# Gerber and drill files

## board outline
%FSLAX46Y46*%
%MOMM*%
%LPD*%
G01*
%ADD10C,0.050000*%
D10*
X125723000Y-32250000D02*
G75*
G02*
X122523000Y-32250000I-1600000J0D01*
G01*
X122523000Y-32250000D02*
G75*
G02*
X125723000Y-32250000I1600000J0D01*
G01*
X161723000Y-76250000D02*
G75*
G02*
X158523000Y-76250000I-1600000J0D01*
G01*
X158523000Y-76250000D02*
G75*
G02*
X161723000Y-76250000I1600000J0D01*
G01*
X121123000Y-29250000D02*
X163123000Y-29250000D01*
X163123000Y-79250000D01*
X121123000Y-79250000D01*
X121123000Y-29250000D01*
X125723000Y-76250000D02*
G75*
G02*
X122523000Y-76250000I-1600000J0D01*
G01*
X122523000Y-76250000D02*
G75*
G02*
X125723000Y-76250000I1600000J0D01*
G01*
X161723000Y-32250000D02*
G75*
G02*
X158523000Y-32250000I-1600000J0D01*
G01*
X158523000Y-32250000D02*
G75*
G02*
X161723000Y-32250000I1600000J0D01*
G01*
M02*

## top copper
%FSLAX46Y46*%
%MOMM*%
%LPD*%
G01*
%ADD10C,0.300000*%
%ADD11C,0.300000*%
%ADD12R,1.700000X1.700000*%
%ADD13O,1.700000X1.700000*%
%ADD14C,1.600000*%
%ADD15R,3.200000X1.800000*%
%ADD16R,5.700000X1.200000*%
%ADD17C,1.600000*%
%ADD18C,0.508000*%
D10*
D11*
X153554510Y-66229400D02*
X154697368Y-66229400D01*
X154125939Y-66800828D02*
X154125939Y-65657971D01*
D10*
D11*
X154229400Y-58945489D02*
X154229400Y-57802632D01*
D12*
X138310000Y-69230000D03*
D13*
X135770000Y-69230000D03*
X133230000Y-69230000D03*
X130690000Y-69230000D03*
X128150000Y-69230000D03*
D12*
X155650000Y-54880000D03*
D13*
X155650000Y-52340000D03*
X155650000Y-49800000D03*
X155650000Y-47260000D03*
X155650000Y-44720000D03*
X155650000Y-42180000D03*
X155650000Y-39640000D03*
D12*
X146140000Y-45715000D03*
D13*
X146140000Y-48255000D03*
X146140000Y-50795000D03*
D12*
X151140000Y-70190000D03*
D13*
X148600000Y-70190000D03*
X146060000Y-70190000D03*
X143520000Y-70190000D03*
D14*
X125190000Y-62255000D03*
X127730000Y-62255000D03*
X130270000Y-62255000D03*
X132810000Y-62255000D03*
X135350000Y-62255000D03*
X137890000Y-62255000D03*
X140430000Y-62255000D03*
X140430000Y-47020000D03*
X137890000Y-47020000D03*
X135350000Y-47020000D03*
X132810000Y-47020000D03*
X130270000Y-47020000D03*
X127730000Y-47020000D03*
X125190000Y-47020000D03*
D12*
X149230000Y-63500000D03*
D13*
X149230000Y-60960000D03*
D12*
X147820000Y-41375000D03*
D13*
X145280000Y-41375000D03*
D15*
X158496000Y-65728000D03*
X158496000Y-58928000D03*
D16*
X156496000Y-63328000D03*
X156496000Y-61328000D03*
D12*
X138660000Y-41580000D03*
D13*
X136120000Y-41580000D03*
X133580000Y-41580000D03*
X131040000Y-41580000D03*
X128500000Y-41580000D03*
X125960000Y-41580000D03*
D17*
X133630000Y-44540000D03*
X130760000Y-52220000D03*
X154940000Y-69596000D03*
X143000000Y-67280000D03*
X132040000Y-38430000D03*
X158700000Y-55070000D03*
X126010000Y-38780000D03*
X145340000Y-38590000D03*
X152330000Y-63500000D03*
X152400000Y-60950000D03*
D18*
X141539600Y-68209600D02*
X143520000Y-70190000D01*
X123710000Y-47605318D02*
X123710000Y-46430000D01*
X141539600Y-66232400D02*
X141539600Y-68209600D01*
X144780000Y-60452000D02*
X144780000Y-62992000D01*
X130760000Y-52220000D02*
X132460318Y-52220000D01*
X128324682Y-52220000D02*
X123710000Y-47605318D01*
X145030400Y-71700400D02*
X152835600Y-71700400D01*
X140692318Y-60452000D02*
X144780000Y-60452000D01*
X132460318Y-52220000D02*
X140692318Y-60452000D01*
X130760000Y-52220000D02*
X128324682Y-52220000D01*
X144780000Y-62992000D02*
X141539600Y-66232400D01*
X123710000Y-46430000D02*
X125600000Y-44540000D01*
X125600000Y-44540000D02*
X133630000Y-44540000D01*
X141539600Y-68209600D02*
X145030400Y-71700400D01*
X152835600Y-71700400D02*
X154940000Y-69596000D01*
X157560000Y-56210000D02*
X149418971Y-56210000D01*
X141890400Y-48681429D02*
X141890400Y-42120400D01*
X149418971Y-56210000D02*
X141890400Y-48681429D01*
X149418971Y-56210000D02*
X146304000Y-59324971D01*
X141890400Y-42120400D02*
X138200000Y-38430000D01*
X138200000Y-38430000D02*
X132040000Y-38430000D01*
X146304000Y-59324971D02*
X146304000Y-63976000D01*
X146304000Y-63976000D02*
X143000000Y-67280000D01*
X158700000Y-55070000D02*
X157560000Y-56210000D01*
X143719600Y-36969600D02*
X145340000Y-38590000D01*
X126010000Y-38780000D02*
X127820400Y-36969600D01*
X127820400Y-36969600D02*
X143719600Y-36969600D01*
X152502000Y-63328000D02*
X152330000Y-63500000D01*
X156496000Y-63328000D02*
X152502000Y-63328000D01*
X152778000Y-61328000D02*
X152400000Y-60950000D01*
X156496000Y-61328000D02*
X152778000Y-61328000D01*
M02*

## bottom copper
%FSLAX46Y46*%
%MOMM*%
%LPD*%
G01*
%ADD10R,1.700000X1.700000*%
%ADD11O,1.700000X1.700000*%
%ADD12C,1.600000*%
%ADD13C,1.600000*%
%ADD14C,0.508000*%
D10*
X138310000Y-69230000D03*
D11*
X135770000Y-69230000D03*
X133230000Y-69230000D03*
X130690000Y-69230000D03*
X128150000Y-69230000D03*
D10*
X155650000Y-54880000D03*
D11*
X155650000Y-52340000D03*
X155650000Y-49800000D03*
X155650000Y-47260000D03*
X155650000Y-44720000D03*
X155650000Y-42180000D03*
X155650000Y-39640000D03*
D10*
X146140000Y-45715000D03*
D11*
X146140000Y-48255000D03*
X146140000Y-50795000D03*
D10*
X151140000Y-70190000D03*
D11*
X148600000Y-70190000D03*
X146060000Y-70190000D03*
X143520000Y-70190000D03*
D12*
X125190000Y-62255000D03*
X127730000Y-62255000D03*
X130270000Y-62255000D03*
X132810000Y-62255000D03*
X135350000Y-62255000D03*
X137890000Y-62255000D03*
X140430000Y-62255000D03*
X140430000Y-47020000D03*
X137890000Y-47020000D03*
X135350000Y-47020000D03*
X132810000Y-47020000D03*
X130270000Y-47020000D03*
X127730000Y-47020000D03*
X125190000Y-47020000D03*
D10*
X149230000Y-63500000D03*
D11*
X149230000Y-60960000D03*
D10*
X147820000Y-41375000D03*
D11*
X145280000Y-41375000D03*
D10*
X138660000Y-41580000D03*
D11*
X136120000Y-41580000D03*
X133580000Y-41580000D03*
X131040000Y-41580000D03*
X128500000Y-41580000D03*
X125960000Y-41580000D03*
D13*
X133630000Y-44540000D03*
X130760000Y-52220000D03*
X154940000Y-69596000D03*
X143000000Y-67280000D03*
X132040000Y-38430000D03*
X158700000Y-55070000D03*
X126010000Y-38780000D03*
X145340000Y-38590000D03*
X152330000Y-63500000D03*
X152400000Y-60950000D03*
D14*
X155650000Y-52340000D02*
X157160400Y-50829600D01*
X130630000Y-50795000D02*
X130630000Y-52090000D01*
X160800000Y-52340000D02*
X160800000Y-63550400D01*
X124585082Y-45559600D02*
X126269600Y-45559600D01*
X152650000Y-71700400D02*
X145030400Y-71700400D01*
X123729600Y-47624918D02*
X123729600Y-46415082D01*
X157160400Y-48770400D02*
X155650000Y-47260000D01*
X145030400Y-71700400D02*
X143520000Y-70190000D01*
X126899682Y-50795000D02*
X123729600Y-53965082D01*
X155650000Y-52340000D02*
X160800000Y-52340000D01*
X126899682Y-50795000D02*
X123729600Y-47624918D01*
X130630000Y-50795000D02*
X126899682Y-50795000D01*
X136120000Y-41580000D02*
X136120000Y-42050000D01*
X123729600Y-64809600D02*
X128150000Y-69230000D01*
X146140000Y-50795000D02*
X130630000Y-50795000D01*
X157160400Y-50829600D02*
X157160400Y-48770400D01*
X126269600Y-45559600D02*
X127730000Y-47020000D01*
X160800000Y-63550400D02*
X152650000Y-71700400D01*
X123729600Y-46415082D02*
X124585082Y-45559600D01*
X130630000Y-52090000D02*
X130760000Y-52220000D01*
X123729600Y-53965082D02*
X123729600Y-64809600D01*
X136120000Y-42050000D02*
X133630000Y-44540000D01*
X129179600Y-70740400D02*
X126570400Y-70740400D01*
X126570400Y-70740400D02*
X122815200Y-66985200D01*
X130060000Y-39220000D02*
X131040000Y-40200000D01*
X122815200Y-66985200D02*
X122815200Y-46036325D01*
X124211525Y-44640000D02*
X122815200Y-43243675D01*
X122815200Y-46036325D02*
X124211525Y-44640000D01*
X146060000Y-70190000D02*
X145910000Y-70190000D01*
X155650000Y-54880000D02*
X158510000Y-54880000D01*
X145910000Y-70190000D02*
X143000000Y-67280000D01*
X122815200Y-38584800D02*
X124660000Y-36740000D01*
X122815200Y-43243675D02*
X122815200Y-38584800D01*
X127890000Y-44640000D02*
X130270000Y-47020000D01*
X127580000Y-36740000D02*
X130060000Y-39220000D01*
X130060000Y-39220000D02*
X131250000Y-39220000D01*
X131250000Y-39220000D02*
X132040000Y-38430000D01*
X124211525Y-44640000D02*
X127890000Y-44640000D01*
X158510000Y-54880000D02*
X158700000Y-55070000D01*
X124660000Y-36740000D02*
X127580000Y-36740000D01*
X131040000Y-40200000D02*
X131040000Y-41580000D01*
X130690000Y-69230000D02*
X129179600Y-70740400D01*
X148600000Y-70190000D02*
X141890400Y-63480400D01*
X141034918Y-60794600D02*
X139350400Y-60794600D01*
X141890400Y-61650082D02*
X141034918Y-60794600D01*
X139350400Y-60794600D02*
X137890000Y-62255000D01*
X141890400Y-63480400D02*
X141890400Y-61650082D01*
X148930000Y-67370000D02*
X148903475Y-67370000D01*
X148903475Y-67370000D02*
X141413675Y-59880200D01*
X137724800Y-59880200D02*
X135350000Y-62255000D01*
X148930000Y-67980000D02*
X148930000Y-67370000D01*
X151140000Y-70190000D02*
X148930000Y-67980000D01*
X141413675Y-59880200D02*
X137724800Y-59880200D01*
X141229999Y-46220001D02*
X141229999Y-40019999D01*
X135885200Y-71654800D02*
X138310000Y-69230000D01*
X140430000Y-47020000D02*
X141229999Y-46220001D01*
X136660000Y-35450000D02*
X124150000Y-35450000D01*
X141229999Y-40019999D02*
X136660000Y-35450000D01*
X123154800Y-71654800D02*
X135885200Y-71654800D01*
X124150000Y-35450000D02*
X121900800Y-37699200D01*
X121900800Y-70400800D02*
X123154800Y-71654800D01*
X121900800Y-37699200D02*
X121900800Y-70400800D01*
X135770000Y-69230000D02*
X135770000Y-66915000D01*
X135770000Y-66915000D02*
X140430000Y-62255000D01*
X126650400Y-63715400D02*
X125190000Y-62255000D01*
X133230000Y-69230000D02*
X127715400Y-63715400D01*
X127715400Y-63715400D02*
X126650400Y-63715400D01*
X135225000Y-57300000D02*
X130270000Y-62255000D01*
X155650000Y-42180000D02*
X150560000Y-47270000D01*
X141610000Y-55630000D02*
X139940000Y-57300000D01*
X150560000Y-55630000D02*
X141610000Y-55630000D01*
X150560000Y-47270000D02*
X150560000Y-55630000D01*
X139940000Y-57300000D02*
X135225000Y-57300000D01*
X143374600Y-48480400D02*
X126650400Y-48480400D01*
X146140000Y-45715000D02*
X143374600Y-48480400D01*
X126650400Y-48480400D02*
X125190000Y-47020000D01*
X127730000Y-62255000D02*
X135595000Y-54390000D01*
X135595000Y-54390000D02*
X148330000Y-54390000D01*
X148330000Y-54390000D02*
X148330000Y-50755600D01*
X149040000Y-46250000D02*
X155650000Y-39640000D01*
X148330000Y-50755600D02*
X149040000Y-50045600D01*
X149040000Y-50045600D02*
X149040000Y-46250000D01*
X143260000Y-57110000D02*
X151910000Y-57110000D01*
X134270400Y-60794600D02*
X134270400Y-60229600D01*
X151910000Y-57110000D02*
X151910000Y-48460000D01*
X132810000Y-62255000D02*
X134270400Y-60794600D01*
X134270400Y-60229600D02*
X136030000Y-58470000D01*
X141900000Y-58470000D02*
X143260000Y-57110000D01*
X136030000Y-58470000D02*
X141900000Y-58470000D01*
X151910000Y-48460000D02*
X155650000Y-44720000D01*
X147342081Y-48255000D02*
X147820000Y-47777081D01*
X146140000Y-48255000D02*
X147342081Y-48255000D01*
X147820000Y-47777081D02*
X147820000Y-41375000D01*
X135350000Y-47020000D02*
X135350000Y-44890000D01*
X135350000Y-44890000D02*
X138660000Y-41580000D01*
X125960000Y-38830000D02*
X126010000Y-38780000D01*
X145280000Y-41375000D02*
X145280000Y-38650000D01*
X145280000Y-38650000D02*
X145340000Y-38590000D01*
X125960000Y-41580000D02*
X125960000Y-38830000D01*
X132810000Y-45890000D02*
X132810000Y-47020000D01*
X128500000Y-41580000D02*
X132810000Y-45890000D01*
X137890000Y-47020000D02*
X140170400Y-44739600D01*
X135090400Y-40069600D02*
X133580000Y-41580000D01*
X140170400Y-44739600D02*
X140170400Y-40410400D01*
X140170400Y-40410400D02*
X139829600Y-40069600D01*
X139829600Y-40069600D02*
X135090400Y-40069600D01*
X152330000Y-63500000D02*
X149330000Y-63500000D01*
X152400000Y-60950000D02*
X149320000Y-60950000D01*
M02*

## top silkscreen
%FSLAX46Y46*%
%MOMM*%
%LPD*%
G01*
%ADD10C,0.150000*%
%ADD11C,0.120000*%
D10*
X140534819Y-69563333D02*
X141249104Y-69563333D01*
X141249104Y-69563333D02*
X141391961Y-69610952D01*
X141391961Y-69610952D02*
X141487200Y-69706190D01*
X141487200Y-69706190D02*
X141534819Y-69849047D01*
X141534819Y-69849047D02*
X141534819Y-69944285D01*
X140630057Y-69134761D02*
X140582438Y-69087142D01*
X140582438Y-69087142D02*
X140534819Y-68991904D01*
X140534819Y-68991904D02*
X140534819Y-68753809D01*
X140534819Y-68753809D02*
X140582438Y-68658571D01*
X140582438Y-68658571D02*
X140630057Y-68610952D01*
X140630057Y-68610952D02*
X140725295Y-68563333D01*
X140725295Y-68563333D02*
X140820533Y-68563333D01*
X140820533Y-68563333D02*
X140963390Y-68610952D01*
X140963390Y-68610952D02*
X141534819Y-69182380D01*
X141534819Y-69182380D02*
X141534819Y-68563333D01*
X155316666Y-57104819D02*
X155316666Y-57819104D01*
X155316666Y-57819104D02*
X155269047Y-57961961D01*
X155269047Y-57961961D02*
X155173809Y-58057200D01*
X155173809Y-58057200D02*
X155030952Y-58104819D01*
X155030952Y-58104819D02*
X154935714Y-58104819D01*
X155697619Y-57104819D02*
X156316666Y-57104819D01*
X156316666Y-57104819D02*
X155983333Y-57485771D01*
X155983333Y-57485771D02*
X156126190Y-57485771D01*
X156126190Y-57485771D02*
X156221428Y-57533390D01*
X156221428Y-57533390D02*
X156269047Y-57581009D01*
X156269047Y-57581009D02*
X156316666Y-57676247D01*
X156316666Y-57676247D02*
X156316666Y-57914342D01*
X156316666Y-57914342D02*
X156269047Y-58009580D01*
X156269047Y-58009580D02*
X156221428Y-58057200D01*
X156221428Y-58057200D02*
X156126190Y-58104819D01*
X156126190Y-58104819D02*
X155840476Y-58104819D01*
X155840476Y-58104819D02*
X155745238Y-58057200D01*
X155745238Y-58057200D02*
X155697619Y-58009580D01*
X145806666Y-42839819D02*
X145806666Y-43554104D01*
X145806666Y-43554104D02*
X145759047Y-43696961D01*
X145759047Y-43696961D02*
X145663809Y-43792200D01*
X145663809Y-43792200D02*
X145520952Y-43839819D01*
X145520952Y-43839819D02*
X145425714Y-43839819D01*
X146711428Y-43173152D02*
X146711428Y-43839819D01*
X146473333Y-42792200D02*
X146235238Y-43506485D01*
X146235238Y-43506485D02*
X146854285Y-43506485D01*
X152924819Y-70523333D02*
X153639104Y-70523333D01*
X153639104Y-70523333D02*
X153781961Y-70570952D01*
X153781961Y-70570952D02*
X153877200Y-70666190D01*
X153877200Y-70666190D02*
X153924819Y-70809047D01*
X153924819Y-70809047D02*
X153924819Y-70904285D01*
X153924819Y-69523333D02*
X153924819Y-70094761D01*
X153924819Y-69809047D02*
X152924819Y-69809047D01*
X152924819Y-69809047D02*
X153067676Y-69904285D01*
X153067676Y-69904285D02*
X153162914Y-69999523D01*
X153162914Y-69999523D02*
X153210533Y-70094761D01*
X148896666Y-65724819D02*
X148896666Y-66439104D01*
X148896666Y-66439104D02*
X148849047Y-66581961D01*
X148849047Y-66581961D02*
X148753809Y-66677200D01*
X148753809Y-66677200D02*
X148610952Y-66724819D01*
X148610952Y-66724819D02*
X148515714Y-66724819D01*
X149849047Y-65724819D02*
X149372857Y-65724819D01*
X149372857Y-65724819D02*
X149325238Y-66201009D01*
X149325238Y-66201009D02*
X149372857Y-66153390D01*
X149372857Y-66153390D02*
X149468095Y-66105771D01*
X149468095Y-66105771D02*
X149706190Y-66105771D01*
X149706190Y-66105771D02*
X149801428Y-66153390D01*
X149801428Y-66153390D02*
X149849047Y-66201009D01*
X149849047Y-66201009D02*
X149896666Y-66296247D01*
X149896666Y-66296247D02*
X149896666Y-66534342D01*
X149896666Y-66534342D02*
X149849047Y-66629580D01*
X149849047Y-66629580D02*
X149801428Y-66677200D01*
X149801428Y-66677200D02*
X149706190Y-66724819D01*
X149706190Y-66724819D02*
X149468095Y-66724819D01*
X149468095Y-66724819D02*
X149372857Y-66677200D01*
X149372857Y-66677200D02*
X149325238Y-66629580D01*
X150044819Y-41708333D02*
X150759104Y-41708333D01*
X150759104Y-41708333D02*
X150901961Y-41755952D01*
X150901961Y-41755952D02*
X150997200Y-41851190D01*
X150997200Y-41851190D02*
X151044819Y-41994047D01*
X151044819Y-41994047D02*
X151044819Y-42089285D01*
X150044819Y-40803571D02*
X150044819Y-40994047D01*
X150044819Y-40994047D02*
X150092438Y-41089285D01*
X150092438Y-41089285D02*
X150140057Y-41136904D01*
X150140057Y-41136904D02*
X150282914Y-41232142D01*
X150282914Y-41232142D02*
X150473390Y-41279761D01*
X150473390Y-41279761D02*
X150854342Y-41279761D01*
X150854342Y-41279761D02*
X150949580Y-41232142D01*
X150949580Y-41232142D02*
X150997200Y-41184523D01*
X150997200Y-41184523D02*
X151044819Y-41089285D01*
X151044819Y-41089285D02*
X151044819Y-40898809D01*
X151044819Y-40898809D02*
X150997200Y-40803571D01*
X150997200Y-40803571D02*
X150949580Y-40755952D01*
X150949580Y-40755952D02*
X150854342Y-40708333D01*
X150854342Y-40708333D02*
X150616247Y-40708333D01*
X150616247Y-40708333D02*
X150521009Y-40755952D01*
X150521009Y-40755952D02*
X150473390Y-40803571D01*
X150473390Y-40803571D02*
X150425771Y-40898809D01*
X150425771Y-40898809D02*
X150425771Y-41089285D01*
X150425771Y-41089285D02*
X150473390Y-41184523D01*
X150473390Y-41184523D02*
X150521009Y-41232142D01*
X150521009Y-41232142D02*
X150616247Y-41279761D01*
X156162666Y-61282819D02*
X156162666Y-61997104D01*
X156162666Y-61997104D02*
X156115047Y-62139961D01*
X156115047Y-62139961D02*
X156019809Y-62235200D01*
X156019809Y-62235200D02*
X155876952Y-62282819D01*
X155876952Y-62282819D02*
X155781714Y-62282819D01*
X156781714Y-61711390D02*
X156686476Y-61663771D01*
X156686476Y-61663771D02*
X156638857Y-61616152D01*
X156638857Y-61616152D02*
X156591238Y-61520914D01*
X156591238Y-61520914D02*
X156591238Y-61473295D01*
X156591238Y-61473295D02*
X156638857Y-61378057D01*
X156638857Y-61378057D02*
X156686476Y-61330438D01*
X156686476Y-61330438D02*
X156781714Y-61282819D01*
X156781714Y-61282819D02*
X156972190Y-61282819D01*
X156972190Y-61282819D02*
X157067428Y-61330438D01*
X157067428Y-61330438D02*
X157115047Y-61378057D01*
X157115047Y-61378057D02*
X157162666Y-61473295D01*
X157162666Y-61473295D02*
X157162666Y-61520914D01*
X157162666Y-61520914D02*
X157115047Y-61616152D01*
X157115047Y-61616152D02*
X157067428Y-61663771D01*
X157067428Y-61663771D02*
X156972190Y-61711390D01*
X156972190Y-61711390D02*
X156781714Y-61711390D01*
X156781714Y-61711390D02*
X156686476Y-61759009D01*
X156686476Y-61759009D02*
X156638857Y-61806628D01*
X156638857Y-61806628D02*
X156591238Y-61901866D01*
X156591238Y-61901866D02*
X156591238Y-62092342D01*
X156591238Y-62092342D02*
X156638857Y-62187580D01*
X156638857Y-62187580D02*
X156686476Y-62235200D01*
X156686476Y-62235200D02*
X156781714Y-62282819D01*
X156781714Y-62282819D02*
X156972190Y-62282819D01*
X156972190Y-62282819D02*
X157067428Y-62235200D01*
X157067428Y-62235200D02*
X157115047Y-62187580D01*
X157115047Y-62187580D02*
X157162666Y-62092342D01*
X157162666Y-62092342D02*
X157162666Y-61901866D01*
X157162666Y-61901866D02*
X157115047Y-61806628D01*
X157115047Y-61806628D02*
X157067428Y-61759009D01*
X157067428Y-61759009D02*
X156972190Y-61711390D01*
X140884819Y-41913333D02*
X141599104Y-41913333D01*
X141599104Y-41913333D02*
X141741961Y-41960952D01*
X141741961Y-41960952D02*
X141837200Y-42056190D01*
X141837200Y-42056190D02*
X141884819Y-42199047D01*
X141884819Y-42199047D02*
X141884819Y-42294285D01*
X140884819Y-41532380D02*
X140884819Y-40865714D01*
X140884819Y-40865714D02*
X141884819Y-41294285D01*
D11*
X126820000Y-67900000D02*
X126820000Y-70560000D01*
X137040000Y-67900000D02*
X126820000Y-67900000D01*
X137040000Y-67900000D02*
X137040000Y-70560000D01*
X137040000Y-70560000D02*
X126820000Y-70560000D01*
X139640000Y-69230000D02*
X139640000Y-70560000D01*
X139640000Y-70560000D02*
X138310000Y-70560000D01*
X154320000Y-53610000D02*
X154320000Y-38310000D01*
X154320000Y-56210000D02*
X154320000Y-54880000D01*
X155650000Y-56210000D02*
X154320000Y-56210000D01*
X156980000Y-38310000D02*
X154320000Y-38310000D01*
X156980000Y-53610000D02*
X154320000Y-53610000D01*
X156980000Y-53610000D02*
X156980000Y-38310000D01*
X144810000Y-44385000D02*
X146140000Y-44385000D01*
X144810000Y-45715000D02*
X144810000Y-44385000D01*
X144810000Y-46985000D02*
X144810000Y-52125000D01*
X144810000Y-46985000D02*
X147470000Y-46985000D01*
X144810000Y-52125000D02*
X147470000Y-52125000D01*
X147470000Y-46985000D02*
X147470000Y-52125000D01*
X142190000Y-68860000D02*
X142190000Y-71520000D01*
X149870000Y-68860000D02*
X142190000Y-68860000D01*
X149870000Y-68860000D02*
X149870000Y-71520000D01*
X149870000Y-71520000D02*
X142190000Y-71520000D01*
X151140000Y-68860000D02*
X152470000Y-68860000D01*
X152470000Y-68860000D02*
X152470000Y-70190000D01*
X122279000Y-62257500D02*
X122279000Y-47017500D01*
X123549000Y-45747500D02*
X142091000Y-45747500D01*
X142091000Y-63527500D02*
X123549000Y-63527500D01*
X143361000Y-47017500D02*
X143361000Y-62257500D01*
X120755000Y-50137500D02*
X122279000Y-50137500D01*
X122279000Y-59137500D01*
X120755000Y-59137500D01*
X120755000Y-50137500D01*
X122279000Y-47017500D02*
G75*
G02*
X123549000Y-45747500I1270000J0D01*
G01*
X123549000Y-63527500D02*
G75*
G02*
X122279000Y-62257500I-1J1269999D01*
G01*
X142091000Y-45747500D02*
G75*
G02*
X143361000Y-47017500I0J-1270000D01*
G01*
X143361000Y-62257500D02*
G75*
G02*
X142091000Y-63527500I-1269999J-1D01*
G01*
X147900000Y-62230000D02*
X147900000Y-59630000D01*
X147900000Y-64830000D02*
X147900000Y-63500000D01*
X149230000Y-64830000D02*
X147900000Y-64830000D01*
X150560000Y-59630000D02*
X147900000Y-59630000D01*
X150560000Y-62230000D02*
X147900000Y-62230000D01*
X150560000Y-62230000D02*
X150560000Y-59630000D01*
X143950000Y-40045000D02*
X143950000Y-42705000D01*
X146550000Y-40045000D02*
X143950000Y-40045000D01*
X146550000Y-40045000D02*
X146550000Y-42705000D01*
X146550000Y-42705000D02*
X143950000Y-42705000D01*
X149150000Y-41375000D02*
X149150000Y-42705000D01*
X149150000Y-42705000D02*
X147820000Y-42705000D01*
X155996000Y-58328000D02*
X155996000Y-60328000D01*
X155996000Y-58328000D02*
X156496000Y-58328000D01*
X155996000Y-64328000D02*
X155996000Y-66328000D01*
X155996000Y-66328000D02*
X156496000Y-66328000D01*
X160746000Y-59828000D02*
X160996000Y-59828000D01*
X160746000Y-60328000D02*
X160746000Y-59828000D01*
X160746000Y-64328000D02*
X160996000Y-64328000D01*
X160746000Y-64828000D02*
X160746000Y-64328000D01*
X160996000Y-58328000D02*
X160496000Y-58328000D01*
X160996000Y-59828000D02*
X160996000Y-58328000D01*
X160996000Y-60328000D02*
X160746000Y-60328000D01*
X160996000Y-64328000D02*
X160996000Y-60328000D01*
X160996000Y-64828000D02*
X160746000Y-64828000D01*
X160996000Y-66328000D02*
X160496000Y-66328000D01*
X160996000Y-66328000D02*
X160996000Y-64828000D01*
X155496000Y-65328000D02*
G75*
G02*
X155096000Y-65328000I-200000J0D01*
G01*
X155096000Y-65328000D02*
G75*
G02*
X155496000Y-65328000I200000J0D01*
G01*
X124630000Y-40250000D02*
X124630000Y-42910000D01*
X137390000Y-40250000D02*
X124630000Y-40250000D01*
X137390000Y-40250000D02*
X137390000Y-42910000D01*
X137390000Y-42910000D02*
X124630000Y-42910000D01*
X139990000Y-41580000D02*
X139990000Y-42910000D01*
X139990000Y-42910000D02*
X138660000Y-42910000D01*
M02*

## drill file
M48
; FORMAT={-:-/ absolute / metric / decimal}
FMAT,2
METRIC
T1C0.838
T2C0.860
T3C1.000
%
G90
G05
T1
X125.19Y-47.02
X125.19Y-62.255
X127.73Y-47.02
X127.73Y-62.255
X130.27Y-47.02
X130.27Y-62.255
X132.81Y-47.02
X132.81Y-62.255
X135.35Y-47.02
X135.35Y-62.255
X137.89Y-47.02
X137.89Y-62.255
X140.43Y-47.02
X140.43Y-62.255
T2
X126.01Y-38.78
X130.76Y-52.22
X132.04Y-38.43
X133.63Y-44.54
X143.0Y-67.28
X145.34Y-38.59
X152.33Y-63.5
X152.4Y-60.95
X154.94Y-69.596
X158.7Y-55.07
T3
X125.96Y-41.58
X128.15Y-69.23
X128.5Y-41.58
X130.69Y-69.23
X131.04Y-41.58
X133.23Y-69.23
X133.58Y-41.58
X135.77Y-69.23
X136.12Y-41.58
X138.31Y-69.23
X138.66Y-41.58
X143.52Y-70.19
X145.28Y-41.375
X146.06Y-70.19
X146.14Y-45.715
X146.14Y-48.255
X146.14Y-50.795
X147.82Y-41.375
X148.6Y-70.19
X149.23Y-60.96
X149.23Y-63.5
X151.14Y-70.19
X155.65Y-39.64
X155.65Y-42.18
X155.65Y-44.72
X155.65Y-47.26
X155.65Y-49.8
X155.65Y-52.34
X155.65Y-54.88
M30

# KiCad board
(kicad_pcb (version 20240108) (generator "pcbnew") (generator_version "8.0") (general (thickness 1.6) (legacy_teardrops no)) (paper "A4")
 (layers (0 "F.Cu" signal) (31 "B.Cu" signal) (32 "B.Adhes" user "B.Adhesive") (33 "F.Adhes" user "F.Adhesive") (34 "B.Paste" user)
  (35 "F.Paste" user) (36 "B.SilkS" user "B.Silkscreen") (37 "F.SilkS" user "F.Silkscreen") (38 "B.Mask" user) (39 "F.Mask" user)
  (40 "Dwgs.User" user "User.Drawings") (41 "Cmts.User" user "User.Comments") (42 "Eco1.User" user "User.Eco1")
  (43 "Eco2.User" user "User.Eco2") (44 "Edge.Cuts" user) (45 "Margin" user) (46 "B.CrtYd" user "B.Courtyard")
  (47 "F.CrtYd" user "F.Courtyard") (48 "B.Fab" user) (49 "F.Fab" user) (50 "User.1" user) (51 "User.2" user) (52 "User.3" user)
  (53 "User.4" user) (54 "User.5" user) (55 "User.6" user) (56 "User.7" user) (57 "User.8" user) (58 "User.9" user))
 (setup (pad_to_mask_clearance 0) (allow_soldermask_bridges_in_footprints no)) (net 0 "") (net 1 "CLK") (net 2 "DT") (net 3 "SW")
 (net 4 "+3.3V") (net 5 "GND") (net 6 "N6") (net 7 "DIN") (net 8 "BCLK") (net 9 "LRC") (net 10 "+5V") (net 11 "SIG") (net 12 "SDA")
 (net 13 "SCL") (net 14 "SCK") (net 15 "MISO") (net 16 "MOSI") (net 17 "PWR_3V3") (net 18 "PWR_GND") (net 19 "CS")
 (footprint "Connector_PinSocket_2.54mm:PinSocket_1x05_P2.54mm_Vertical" (layer "F.Cu") (at 138.31 69.23 -90)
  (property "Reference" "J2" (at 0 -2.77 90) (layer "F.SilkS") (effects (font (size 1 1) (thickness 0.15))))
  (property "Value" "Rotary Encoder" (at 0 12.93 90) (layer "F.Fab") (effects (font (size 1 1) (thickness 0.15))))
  (fp_line (start -1.33 11.49) (end 1.33 11.49) (stroke (width 0.12) (type solid)) (layer "F.SilkS"))
  (fp_line (start -1.33 1.27) (end -1.33 11.49) (stroke (width 0.12) (type solid)) (layer "F.SilkS"))
  (fp_line (start -1.33 1.27) (end 1.33 1.27) (stroke (width 0.12) (type solid)) (layer "F.SilkS"))
  (fp_line (start 1.33 1.27) (end 1.33 11.49) (stroke (width 0.12) (type solid)) (layer "F.SilkS"))
  (fp_line (start 0 -1.33) (end 1.33 -1.33) (stroke (width 0.12) (type solid)) (layer "F.SilkS"))
  (fp_line (start 1.33 -1.33) (end 1.33 0) (stroke (width 0.12) (type solid)) (layer "F.SilkS"))
  (pad "1" thru_hole rect (at 0 0 270) (size 1.7 1.7) (drill 1) (layers "*.Cu" "*.Mask") (remove_unused_layers no) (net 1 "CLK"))
  (pad "2" thru_hole oval (at 0 2.54 270) (size 1.7 1.7) (drill 1) (layers "*.Cu" "*.Mask") (remove_unused_layers no) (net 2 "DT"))
  (pad "3" thru_hole oval (at 0 5.08 270) (size 1.7 1.7) (drill 1) (layers "*.Cu" "*.Mask") (remove_unused_layers no) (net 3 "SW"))
  (pad "4" thru_hole oval (at 0 7.62 270) (size 1.7 1.7) (drill 1) (layers "*.Cu" "*.Mask") (remove_unused_layers no) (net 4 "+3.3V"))
  (pad "5" thru_hole oval (at 0 10.16 270) (size 1.7 1.7) (drill 1) (layers "*.Cu" "*.Mask") (remove_unused_layers no) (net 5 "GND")))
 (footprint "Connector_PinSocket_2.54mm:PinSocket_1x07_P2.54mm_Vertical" (layer "F.Cu") (at 155.65 54.88 180)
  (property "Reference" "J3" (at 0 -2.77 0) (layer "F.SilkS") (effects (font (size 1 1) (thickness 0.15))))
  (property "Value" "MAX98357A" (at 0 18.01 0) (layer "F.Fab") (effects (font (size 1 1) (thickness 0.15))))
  (fp_line (start 1.33 1.27) (end 1.33 16.57) (stroke (width 0.12) (type solid)) (layer "F.SilkS"))
  (fp_line (start 1.33 -1.33) (end 1.33 0) (stroke (width 0.12) (type solid)) (layer "F.SilkS"))
  (fp_line (start 0 -1.33) (end 1.33 -1.33) (stroke (width 0.12) (type solid)) (layer "F.SilkS"))
  (fp_line (start -1.33 16.57) (end 1.33 16.57) (stroke (width 0.12) (type solid)) (layer "F.SilkS"))
  (fp_line (start -1.33 1.27) (end 1.33 1.27) (stroke (width 0.12) (type solid)) (layer "F.SilkS"))
  (fp_line (start -1.33 1.27) (end -1.33 16.57) (stroke (width 0.12) (type solid)) (layer "F.SilkS"))
  (pad "1" thru_hole rect (at 0 0 180) (size 1.7 1.7) (drill 1) (layers "*.Cu" "*.Mask") (remove_unused_layers no) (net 4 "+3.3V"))
  (pad "2" thru_hole oval (at 0 2.54 180) (size 1.7 1.7) (drill 1) (layers "*.Cu" "*.Mask") (remove_unused_layers no) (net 5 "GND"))
  (pad "3" thru_hole oval (at 0 5.08 180) (size 1.7 1.7) (drill 1) (layers "*.Cu" "*.Mask") (remove_unused_layers no) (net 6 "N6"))
  (pad "4" thru_hole oval (at 0 7.62 180) (size 1.7 1.7) (drill 1) (layers "*.Cu" "*.Mask") (remove_unused_layers no) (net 5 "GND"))
  (pad "5" thru_hole oval (at 0 10.16 180) (size 1.7 1.7) (drill 1) (layers "*.Cu" "*.Mask") (remove_unused_layers no) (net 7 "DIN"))
  (pad "6" thru_hole oval (at 0 12.7 180) (size 1.7 1.7) (drill 1) (layers "*.Cu" "*.Mask") (remove_unused_layers no) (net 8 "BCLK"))
  (pad "7" thru_hole oval (at 0 15.24 180) (size 1.7 1.7) (drill 1) (layers "*.Cu" "*.Mask") (remove_unused_layers no) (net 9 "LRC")))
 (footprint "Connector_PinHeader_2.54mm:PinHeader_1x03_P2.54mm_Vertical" (layer "F.Cu") (at 146.14 45.715)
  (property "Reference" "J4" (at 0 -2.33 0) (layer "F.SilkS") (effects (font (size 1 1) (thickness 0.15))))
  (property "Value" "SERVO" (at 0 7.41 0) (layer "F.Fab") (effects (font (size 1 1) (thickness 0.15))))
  (fp_line (start -1.33 -1.33) (end 0 -1.33) (stroke (width 0.12) (type solid)) (layer "F.SilkS"))
  (fp_line (start -1.33 0) (end -1.33 -1.33) (stroke (width 0.12) (type solid)) (layer "F.SilkS"))
  (fp_line (start -1.33 1.27) (end -1.33 6.41) (stroke (width 0.12) (type solid)) (layer "F.SilkS"))
  (fp_line (start -1.33 1.27) (end 1.33 1.27) (stroke (width 0.12) (type solid)) (layer "F.SilkS"))
  (fp_line (start -1.33 6.41) (end 1.33 6.41) (stroke (width 0.12) (type solid)) (layer "F.SilkS"))
  (fp_line (start 1.33 1.27) (end 1.33 6.41) (stroke (width 0.12) (type solid)) (layer "F.SilkS"))
  (pad "1" thru_hole rect (at 0 0) (size 1.7 1.7) (drill 1) (layers "*.Cu" "*.Mask") (remove_unused_layers no) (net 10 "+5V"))
  (pad "2" thru_hole oval (at 0 2.54) (size 1.7 1.7) (drill 1) (layers "*.Cu" "*.Mask") (remove_unused_layers no) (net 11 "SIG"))
  (pad "3" thru_hole oval (at 0 5.08) (size 1.7 1.7) (drill 1) (layers "*.Cu" "*.Mask") (remove_unused_layers no) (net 5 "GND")))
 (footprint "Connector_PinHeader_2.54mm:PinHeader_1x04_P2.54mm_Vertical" (layer "F.Cu") (at 151.14 70.19 -90)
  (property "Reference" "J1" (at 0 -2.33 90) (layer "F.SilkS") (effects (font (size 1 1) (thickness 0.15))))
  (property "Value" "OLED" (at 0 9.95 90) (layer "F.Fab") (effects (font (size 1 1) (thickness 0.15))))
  (fp_line (start -1.33 8.95) (end 1.33 8.95) (stroke (width 0.12) (type solid)) (layer "F.SilkS"))
  (fp_line (start -1.33 1.27) (end -1.33 8.95) (stroke (width 0.12) (type solid)) (layer "F.SilkS"))
  (fp_line (start -1.33 1.27) (end 1.33 1.27) (stroke (width 0.12) (type solid)) (layer "F.SilkS"))
  (fp_line (start 1.33 1.27) (end 1.33 8.95) (stroke (width 0.12) (type solid)) (layer "F.SilkS"))
  (fp_line (start -1.33 0) (end -1.33 -1.33) (stroke (width 0.12) (type solid)) (layer "F.SilkS"))
  (fp_line (start -1.33 -1.33) (end 0 -1.33) (stroke (width 0.12) (type solid)) (layer "F.SilkS"))
  (pad "1" thru_hole rect (at 0 0 270) (size 1.7 1.7) (drill 1) (layers "*.Cu" "*.Mask") (remove_unused_layers no) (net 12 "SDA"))
  (pad "2" thru_hole oval (at 0 2.54 270) (size 1.7 1.7) (drill 1) (layers "*.Cu" "*.Mask") (remove_unused_layers no) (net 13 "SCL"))
  (pad "3" thru_hole oval (at 0 5.08 270) (size 1.7 1.7) (drill 1) (layers "*.Cu" "*.Mask") (remove_unused_layers no) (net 4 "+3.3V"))
  (pad "4" thru_hole oval (at 0 7.62 270) (size 1.7 1.7) (drill 1) (layers "*.Cu" "*.Mask") (remove_unused_layers no) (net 5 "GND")))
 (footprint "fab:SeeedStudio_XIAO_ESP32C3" (layer "F.Cu") (at 132.81 54.64 90)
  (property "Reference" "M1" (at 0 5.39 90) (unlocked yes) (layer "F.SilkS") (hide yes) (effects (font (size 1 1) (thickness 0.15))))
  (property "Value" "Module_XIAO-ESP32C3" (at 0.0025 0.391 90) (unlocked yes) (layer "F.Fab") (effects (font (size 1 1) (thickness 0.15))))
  (fp_line (start -7.6175 -10.531) (end 7.6225 -10.531) (stroke (width 0.12) (type solid)) (layer "F.SilkS"))
  (fp_line (start 8.8925 -9.261) (end 8.8925 9.281) (stroke (width 0.12) (type solid)) (layer "F.SilkS"))
  (fp_line (start -8.8875 9.281) (end -8.8875 -9.261) (stroke (width 0.12) (type solid)) (layer "F.SilkS"))
  (fp_line (start 7.6225 10.551) (end -7.6175 10.551) (stroke (width 0.12) (type solid)) (layer "F.SilkS"))
  (fp_rect (start -4.4975 -10.531) (end 4.5025 -12.055) (stroke (width 0.12) (type solid)) (fill none) (layer "F.SilkS"))
  (fp_arc (start 7.6225 -10.531) (mid 8.520526 -10.159026) (end 8.8925 -9.261) (stroke (width 0.12) (type solid)) (layer "F.SilkS"))
  (fp_arc (start -8.8875 -9.261) (mid -8.515526 -10.159026) (end -7.6175 -10.531) (stroke (width 0.12) (type solid)) (layer "F.SilkS"))
  (fp_arc (start 8.8925 9.281) (mid 8.520526 10.179026) (end 7.6225 10.551) (stroke (width 0.12) (type solid)) (layer "F.SilkS"))
  (fp_arc (start -7.6175 10.551) (mid -8.515526 10.179026) (end -8.8875 9.281) (stroke (width 0.12) (type solid)) (layer "F.SilkS"))
  (pad "1" thru_hole circle (at -7.615 -7.62 90) (size 1.6 1.6) (drill 0.8382) (layers "*.Cu" "*.Mask") (remove_unused_layers no)
   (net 3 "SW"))
  (pad "2" thru_hole circle (at -7.615 -5.08 90) (size 1.6 1.6) (drill 0.8382) (layers "*.Cu" "*.Mask") (remove_unused_layers no)
   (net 9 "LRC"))
  (pad "3" thru_hole circle (at -7.615 -2.54 90) (size 1.6 1.6) (drill 0.8382) (layers "*.Cu" "*.Mask") (remove_unused_layers no)
   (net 8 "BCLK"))
  (pad "4" thru_hole circle (at -7.615 0 90) (size 1.6 1.6) (drill 0.8382) (layers "*.Cu" "*.Mask") (remove_unused_layers no) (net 7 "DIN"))
  (pad "5" thru_hole circle (at -7.615 2.54 90) (size 1.6 1.6) (drill 0.8382) (layers "*.Cu" "*.Mask") (remove_unused_layers no)
   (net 12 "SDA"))
  (pad "6" thru_hole circle (at -7.615 5.08 90) (size 1.6 1.6) (drill 0.8382) (layers "*.Cu" "*.Mask") (remove_unused_layers no)
   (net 13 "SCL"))
  (pad "7" thru_hole circle (at -7.615 7.62 90) (size 1.6 1.6) (drill 0.8382) (layers "*.Cu" "*.Mask") (remove_unused_layers no)
   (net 2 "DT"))
  (pad "8" thru_hole circle (at 7.62 7.62 90) (size 1.6 1.6) (drill 0.8382) (layers "*.Cu" "*.Mask") (remove_unused_layers no) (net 1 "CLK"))
  (pad "9" thru_hole circle (at 7.62 5.08 90) (size 1.6 1.6) (drill 0.8382) (layers "*.Cu" "*.Mask") (remove_unused_layers no)
   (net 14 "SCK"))
  (pad "10" thru_hole circle (at 7.62 2.54 90) (size 1.6 1.6) (drill 0.8382) (layers "*.Cu" "*.Mask") (remove_unused_layers no)
   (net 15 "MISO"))
  (pad "11" thru_hole circle (at 7.62 0 90) (size 1.6 1.6) (drill 0.8382) (layers "*.Cu" "*.Mask") (remove_unused_layers no) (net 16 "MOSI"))
  (pad "12" thru_hole circle (at 7.62 -2.54 90) (size 1.6 1.6) (drill 0.8382) (layers "*.Cu" "*.Mask") (remove_unused_layers no)
   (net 4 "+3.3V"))
  (pad "13" thru_hole circle (at 7.62 -5.08 90) (size 1.6 1.6) (drill 0.8382) (layers "*.Cu" "*.Mask") (remove_unused_layers no)
   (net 5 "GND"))
  (pad "14" thru_hole circle (at 7.62 -7.62 90) (size 1.6 1.6) (drill 0.8382) (layers "*.Cu" "*.Mask") (remove_unused_layers no)
   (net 10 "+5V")))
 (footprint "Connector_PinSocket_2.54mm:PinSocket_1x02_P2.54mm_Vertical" (layer "F.Cu") (at 149.23 63.5 180)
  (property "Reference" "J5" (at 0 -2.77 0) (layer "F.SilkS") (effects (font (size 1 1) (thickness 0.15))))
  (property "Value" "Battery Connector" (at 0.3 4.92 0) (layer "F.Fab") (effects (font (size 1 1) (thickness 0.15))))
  (fp_line (start 1.33 1.27) (end 1.33 3.87) (stroke (width 0.12) (type solid)) (layer "F.SilkS"))
  (fp_line (start 1.33 -1.33) (end 1.33 0) (stroke (width 0.12) (type solid)) (layer "F.SilkS"))
  (fp_line (start 0 -1.33) (end 1.33 -1.33) (stroke (width 0.12) (type solid)) (layer "F.SilkS"))
  (fp_line (start -1.33 3.87) (end 1.33 3.87) (stroke (width 0.12) (type solid)) (layer "F.SilkS"))
  (fp_line (start -1.33 1.27) (end 1.33 1.27) (stroke (width 0.12) (type solid)) (layer "F.SilkS"))
  (fp_line (start -1.33 1.27) (end -1.33 3.87) (stroke (width 0.12) (type solid)) (layer "F.SilkS"))
  (pad "1" thru_hole rect (at 0 0 180) (size 1.7 1.7) (drill 1) (layers "*.Cu" "*.Mask") (remove_unused_layers no) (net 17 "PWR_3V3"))
  (pad "2" thru_hole oval (at 0 2.54 180) (size 1.7 1.7) (drill 1) (layers "*.Cu" "*.Mask") (remove_unused_layers no) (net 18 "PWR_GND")))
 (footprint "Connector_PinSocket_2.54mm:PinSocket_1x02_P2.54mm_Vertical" (layer "F.Cu") (at 147.82 41.375 -90)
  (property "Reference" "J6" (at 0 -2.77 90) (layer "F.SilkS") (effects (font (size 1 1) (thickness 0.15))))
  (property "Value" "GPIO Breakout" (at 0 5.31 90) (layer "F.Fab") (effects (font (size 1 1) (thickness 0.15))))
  (fp_line (start -1.33 3.87) (end 1.33 3.87) (stroke (width 0.12) (type solid)) (layer "F.SilkS"))
  (fp_line (start -1.33 1.27) (end -1.33 3.87) (stroke (width 0.12) (type solid)) (layer "F.SilkS"))
  (fp_line (start -1.33 1.27) (end 1.33 1.27) (stroke (width 0.12) (type solid)) (layer "F.SilkS"))
  (fp_line (start 1.33 1.27) (end 1.33 3.87) (stroke (width 0.12) (type solid)) (layer "F.SilkS"))
  (fp_line (start 0 -1.33) (end 1.33 -1.33) (stroke (width 0.12) (type solid)) (layer "F.SilkS"))
  (fp_line (start 1.33 -1.33) (end 1.33 0) (stroke (width 0.12) (type solid)) (layer "F.SilkS"))
  (pad "1" thru_hole rect (at 0 0 270) (size 1.7 1.7) (drill 1) (layers "*.Cu" "*.Mask") (remove_unused_layers no) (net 11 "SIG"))
  (pad "2" thru_hole oval (at 0 2.54 270) (size 1.7 1.7) (drill 1) (layers "*.Cu" "*.Mask") (remove_unused_layers no) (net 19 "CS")))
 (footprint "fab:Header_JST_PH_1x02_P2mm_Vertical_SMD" (layer "F.Cu") (at 156.496 62.328 180)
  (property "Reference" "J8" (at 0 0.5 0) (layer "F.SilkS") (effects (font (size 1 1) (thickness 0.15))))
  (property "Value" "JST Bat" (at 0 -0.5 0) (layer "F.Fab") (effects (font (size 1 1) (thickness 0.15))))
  (fp_line (start 0.5 4) (end 0.5 2) (stroke (width 0.12) (type solid)) (layer "F.SilkS"))
  (fp_line (start 0.5 4) (end 0 4) (stroke (width 0.12) (type solid)) (layer "F.SilkS"))
  (fp_line (start 0.5 -2) (end 0.5 -4) (stroke (width 0.12) (type solid)) (layer "F.SilkS"))
  (fp_line (start 0.5 -4) (end 0 -4) (stroke (width 0.12) (type solid)) (layer "F.SilkS"))
  (fp_line (start -4.25 2.5) (end -4.5 2.5) (stroke (width 0.12) (type solid)) (layer "F.SilkS"))
  (fp_line (start -4.25 2) (end -4.25 2.5) (stroke (width 0.12) (type solid)) (layer "F.SilkS"))
  (fp_line (start -4.25 -2) (end -4.5 -2) (stroke (width 0.12) (type solid)) (layer "F.SilkS"))
  (fp_line (start -4.25 -2.5) (end -4.25 -2) (stroke (width 0.12) (type solid)) (layer "F.SilkS"))
  (fp_line (start -4.5 4) (end -4 4) (stroke (width 0.12) (type solid)) (layer "F.SilkS"))
  (fp_line (start -4.5 2.5) (end -4.5 4) (stroke (width 0.12) (type solid)) (layer "F.SilkS"))
  (fp_line (start -4.5 2) (end -4.25 2) (stroke (width 0.12) (type solid)) (layer "F.SilkS"))
  (fp_line (start -4.5 -2) (end -4.5 2) (stroke (width 0.12) (type solid)) (layer "F.SilkS"))
  (fp_line (start -4.5 -2.5) (end -4.25 -2.5) (stroke (width 0.12) (type solid)) (layer "F.SilkS"))
  (fp_line (start -4.5 -4) (end -4 -4) (stroke (width 0.12) (type solid)) (layer "F.SilkS"))
  (fp_line (start -4.5 -4) (end -4.5 -2.5) (stroke (width 0.12) (type solid)) (layer "F.SilkS"))
  (fp_circle (center 1.2 -3) (end 1.4 -3) (stroke (width 0.12) (type solid)) (fill none) (layer "F.SilkS"))
  (pad "" smd rect (at -2 -3.4 180) (size 3.2 1.8) (layers "F.Cu" "F.Paste" "F.Mask"))
  (pad "" smd rect (at -2 3.4 180) (size 3.2 1.8) (layers "F.Cu" "F.Paste" "F.Mask"))
  (pad "1" smd rect (at 0 -1 180) (size 5.7 1.2) (layers "F.Cu" "F.Paste" "F.Mask") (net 17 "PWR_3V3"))
  (pad "2" smd rect (at 0 1 180) (size 5.7 1.2) (layers "F.Cu" "F.Paste" "F.Mask") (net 18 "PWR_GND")))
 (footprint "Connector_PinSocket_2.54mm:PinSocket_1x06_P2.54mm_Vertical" (layer "F.Cu") (at 138.66 41.58 -90)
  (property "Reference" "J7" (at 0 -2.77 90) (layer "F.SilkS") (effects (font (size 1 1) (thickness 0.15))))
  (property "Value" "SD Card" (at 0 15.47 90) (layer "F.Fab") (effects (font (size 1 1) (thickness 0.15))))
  (fp_line (start -1.33 14.03) (end 1.33 14.03) (stroke (width 0.12) (type solid)) (layer "F.SilkS"))
  (fp_line (start -1.33 1.27) (end -1.33 14.03) (stroke (width 0.12) (type solid)) (layer "F.SilkS"))
  (fp_line (start -1.33 1.27) (end 1.33 1.27) (stroke (width 0.12) (type solid)) (layer "F.SilkS"))
  (fp_line (start 1.33 1.27) (end 1.33 14.03) (stroke (width 0.12) (type solid)) (layer "F.SilkS"))
  (fp_line (start 0 -1.33) (end 1.33 -1.33) (stroke (width 0.12) (type solid)) (layer "F.SilkS"))
  (fp_line (start 1.33 -1.33) (end 1.33 0) (stroke (width 0.12) (type solid)) (layer "F.SilkS"))
  (pad "1" thru_hole rect (at 0 0 270) (size 1.7 1.7) (drill 1) (layers "*.Cu" "*.Mask") (remove_unused_layers no) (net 15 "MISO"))
  (pad "2" thru_hole oval (at 0 2.54 270) (size 1.7 1.7) (drill 1) (layers "*.Cu" "*.Mask") (remove_unused_layers no) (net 5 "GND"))
  (pad "3" thru_hole oval (at 0 5.08 270) (size 1.7 1.7) (drill 1) (layers "*.Cu" "*.Mask") (remove_unused_layers no) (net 14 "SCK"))
  (pad "4" thru_hole oval (at 0 7.62 270) (size 1.7 1.7) (drill 1) (layers "*.Cu" "*.Mask") (remove_unused_layers no) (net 4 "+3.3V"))
  (pad "5" thru_hole oval (at 0 10.16 270) (size 1.7 1.7) (drill 1) (layers "*.Cu" "*.Mask") (remove_unused_layers no) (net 16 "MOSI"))
  (pad "6" thru_hole oval (at 0 12.7 270) (size 1.7 1.7) (drill 1) (layers "*.Cu" "*.Mask") (remove_unused_layers no) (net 19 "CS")))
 (gr_circle (center 124.123 32.25) (end 125.723 32.25) (stroke (width 0.05) (type default)) (fill none) (layer "Edge.Cuts"))
 (gr_circle (center 160.123 76.25) (end 161.723 76.25) (stroke (width 0.05) (type default)) (fill none) (layer "Edge.Cuts"))
 (gr_rect (start 121.123 29.25) (end 163.123 79.25) (stroke (width 0.05) (type default)) (fill none) (layer "Edge.Cuts"))
 (gr_circle (center 124.123 76.25) (end 125.723 76.25) (stroke (width 0.05) (type default)) (fill none) (layer "Edge.Cuts"))
 (gr_circle (center 160.123 32.25) (end 161.723 32.25) (stroke (width 0.05) (type default)) (fill none) (layer "Edge.Cuts"))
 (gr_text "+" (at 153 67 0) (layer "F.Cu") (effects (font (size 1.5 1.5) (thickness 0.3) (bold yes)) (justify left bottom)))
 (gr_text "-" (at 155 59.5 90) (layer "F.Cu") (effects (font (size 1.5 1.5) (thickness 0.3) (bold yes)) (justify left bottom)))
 (segment (start 141.5396 68.2096) (end 143.52 70.19) (width 0.508) (layer "F.Cu") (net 5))
 (segment (start 123.71 47.605318) (end 123.71 46.43) (width 0.508) (layer "F.Cu") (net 5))
 (segment (start 141.5396 66.2324) (end 141.5396 68.2096) (width 0.508) (layer "F.Cu") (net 5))
 (segment (start 144.78 60.452) (end 144.78 62.992) (width 0.508) (layer "F.Cu") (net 5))
 (segment (start 130.76 52.22) (end 132.460318 52.22) (width 0.508) (layer "F.Cu") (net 5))
 (segment (start 128.324682 52.22) (end 123.71 47.605318) (width 0.508) (layer "F.Cu") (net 5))
 (segment (start 145.0304 71.7004) (end 152.8356 71.7004) (width 0.508) (layer "F.Cu") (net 5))
 (segment (start 140.692318 60.452) (end 144.78 60.452) (width 0.508) (layer "F.Cu") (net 5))
 (segment (start 132.460318 52.22) (end 140.692318 60.452) (width 0.508) (layer "F.Cu") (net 5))
 (segment (start 130.76 52.22) (end 128.324682 52.22) (width 0.508) (layer "F.Cu") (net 5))
 (segment (start 144.78 62.992) (end 141.5396 66.2324) (width 0.508) (layer "F.Cu") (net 5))
 (segment (start 123.71 46.43) (end 125.6 44.54) (width 0.508) (layer "F.Cu") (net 5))
 (segment (start 125.6 44.54) (end 133.63 44.54) (width 0.508) (layer "F.Cu") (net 5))
 (segment (start 141.5396 68.2096) (end 145.0304 71.7004) (width 0.508) (layer "F.Cu") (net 5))
 (segment (start 152.8356 71.7004) (end 154.94 69.596) (width 0.508) (layer "F.Cu") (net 5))
 (via (at 133.63 44.54) (size 1.6) (drill 0.86) (layers "F.Cu" "B.Cu") (free yes) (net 5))
 (via (at 130.76 52.22) (size 1.6) (drill 0.86) (layers "F.Cu" "B.Cu") (free yes) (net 5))
 (via (at 154.94 69.596) (size 1.6) (drill 0.86) (layers "F.Cu" "B.Cu") (free yes) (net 5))
 (segment (start 155.65 52.34) (end 157.1604 50.8296) (width 0.508) (layer "B.Cu") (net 5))
 (segment (start 130.63 50.795) (end 130.63 52.09) (width 0.508) (layer "B.Cu") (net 5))
 (segment (start 160.8 52.34) (end 160.8 63.5504) (width 0.508) (layer "B.Cu") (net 5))
 (segment (start 124.585082 45.5596) (end 126.2696 45.5596) (width 0.508) (layer "B.Cu") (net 5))
 (segment (start 152.65 71.7004) (end 145.0304 71.7004) (width 0.508) (layer "B.Cu") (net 5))
 (segment (start 123.7296 47.624918) (end 123.7296 46.415082) (width 0.508) (layer "B.Cu") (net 5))
 (segment (start 157.1604 48.7704) (end 155.65 47.26) (width 0.508) (layer "B.Cu") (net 5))
 (segment (start 145.0304 71.7004) (end 143.52 70.19) (width 0.508) (layer "B.Cu") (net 5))
 (segment (start 126.899682 50.795) (end 123.7296 53.965082) (width 0.508) (layer "B.Cu") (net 5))
 (segment (start 155.65 52.34) (end 160.8 52.34) (width 0.508) (layer "B.Cu") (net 5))
 (segment (start 126.899682 50.795) (end 123.7296 47.624918) (width 0.508) (layer "B.Cu") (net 5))
 (segment (start 130.63 50.795) (end 126.899682 50.795) (width 0.508) (layer "B.Cu") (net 5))
 (segment (start 136.12 41.58) (end 136.12 42.05) (width 0.508) (layer "B.Cu") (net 5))
 (segment (start 123.7296 64.8096) (end 128.15 69.23) (width 0.508) (layer "B.Cu") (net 5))
 (segment (start 146.14 50.795) (end 130.63 50.795) (width 0.508) (layer "B.Cu") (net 5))
 (segment (start 157.1604 50.8296) (end 157.1604 48.7704) (width 0.508) (layer "B.Cu") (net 5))
 (segment (start 126.2696 45.5596) (end 127.73 47.02) (width 0.508) (layer "B.Cu") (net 5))
 (segment (start 160.8 63.5504) (end 152.65 71.7004) (width 0.508) (layer "B.Cu") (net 5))
 (segment (start 123.7296 46.415082) (end 124.585082 45.5596) (width 0.508) (layer "B.Cu") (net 5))
 (segment (start 130.63 52.09) (end 130.76 52.22) (width 0.508) (layer "B.Cu") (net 5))
 (segment (start 123.7296 53.965082) (end 123.7296 64.8096) (width 0.508) (layer "B.Cu") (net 5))
 (segment (start 136.12 42.05) (end 133.63 44.54) (width 0.508) (layer "B.Cu") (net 5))
 (segment (start 157.56 56.21) (end 149.418971 56.21) (width 0.508) (layer "F.Cu") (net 4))
 (segment (start 141.8904 48.681429) (end 141.8904 42.1204) (width 0.508) (layer "F.Cu") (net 4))
 (segment (start 149.418971 56.21) (end 141.8904 48.681429) (width 0.508) (layer "F.Cu") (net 4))
 (segment (start 149.418971 56.21) (end 146.304 59.324971) (width 0.508) (layer "F.Cu") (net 4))
 (segment (start 141.8904 42.1204) (end 138.2 38.43) (width 0.508) (layer "F.Cu") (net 4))
 (segment (start 138.2 38.43) (end 132.04 38.43) (width 0.508) (layer "F.Cu") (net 4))
 (segment (start 146.304 59.324971) (end 146.304 63.976) (width 0.508) (layer "F.Cu") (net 4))
 (segment (start 146.304 63.976) (end 143 67.28) (width 0.508) (layer "F.Cu") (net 4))
 (segment (start 158.7 55.07) (end 157.56 56.21) (width 0.508) (layer "F.Cu") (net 4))
 (via (at 143 67.28) (size 1.6) (drill 0.86) (layers "F.Cu" "B.Cu") (free yes) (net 4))
 (via (at 132.04 38.43) (size 1.6) (drill 0.86) (layers "F.Cu" "B.Cu") (free yes) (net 4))
 (via (at 158.7 55.07) (size 1.6) (drill 0.86) (layers "F.Cu" "B.Cu") (free yes) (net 4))
 (segment (start 129.1796 70.7404) (end 126.5704 70.7404) (width 0.508) (layer "B.Cu") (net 4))
 (segment (start 126.5704 70.7404) (end 122.8152 66.9852) (width 0.508) (layer "B.Cu") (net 4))
 (segment (start 130.06 39.22) (end 131.04 40.2) (width 0.508) (layer "B.Cu") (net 4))
 (segment (start 122.8152 66.9852) (end 122.8152 46.036325) (width 0.508) (layer "B.Cu") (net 4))
 (segment (start 124.211525 44.64) (end 122.8152 43.243675) (width 0.508) (layer "B.Cu") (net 4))
 (segment (start 122.8152 46.036325) (end 124.211525 44.64) (width 0.508) (layer "B.Cu") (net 4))
 (segment (start 146.06 70.19) (end 145.91 70.19) (width 0.508) (layer "B.Cu") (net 4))
 (segment (start 155.65 54.88) (end 158.51 54.88) (width 0.508) (layer "B.Cu") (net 4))
 (segment (start 145.91 70.19) (end 143 67.28) (width 0.508) (layer "B.Cu") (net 4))
 (segment (start 122.8152 38.5848) (end 124.66 36.74) (width 0.508) (layer "B.Cu") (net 4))
 (segment (start 122.8152 43.243675) (end 122.8152 38.5848) (width 0.508) (layer "B.Cu") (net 4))
 (segment (start 127.89 44.64) (end 130.27 47.02) (width 0.508) (layer "B.Cu") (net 4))
 (segment (start 127.58 36.74) (end 130.06 39.22) (width 0.508) (layer "B.Cu") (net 4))
 (segment (start 130.06 39.22) (end 131.25 39.22) (width 0.508) (layer "B.Cu") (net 4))
 (segment (start 131.25 39.22) (end 132.04 38.43) (width 0.508) (layer "B.Cu") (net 4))
 (segment (start 124.211525 44.64) (end 127.89 44.64) (width 0.508) (layer "B.Cu") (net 4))
 (segment (start 158.51 54.88) (end 158.7 55.07) (width 0.508) (layer "B.Cu") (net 4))
 (segment (start 124.66 36.74) (end 127.58 36.74) (width 0.508) (layer "B.Cu") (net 4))
 (segment (start 131.04 40.2) (end 131.04 41.58) (width 0.508) (layer "B.Cu") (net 4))
 (segment (start 130.69 69.23) (end 129.1796 70.7404) (width 0.508) (layer "B.Cu") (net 4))
 (segment (start 148.6 70.19) (end 141.8904 63.4804) (width 0.508) (layer "B.Cu") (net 13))
 (segment (start 141.034918 60.7946) (end 139.3504 60.7946) (width 0.508) (layer "B.Cu") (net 13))
 (segment (start 141.8904 61.650082) (end 141.034918 60.7946) (width 0.508) (layer "B.Cu") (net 13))
 (segment (start 139.3504 60.7946) (end 137.89 62.255) (width 0.508) (layer "B.Cu") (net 13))
 (segment (start 141.8904 63.4804) (end 141.8904 61.650082) (width 0.508) (layer "B.Cu") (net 13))
 (segment (start 148.93 67.37) (end 148.903475 67.37) (width 0.508) (layer "B.Cu") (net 12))
 (segment (start 148.903475 67.37) (end 141.413675 59.8802) (width 0.508) (layer "B.Cu") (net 12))
 (segment (start 137.7248 59.8802) (end 135.35 62.255) (width 0.508) (layer "B.Cu") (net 12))
 (segment (start 148.93 67.98) (end 148.93 67.37) (width 0.508) (layer "B.Cu") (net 12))
 (segment (start 151.14 70.19) (end 148.93 67.98) (width 0.508) (layer "B.Cu") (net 12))
 (segment (start 141.413675 59.8802) (end 137.7248 59.8802) (width 0.508) (layer "B.Cu") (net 12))
 (segment (start 141.229999 46.220001) (end 141.229999 40.019999) (width 0.508) (layer "B.Cu") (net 1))
 (segment (start 135.8852 71.6548) (end 138.31 69.23) (width 0.508) (layer "B.Cu") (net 1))
 (segment (start 140.43 47.02) (end 141.229999 46.220001) (width 0.508) (layer "B.Cu") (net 1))
 (segment (start 136.66 35.45) (end 124.15 35.45) (width 0.508) (layer "B.Cu") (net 1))
 (segment (start 141.229999 40.019999) (end 136.66 35.45) (width 0.508) (layer "B.Cu") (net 1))
 (segment (start 123.1548 71.6548) (end 135.8852 71.6548) (width 0.508) (layer "B.Cu") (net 1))
 (segment (start 124.15 35.45) (end 121.9008 37.6992) (width 0.508) (layer "B.Cu") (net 1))
 (segment (start 121.9008 70.4008) (end 123.1548 71.6548) (width 0.508) (layer "B.Cu") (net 1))
 (segment (start 121.9008 37.6992) (end 121.9008 70.4008) (width 0.508) (layer "B.Cu") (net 1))
 (segment (start 135.77 69.23) (end 135.77 66.915) (width 0.508) (layer "B.Cu") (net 2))
 (segment (start 135.77 66.915) (end 140.43 62.255) (width 0.508) (layer "B.Cu") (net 2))
 (segment (start 126.6504 63.7154) (end 125.19 62.255) (width 0.508) (layer "B.Cu") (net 3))
 (segment (start 133.23 69.23) (end 127.7154 63.7154) (width 0.508) (layer "B.Cu") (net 3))
 (segment (start 127.7154 63.7154) (end 126.6504 63.7154) (width 0.508) (layer "B.Cu") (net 3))
 (segment (start 135.225 57.3) (end 130.27 62.255) (width 0.508) (layer "B.Cu") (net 8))
 (segment (start 155.65 42.18) (end 150.56 47.27) (width 0.508) (layer "B.Cu") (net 8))
 (segment (start 141.61 55.63) (end 139.94 57.3) (width 0.508) (layer "B.Cu") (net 8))
 (segment (start 150.56 55.63) (end 141.61 55.63) (width 0.508) (layer "B.Cu") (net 8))
 (segment (start 150.56 47.27) (end 150.56 55.63) (width 0.508) (layer "B.Cu") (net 8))
 (segment (start 139.94 57.3) (end 135.225 57.3) (width 0.508) (layer "B.Cu") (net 8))
 (segment (start 143.3746 48.4804) (end 126.6504 48.4804) (width 0.508) (layer "B.Cu") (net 10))
 (segment (start 146.14 45.715) (end 143.3746 48.4804) (width 0.508) (layer "B.Cu") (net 10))
 (segment (start 126.6504 48.4804) (end 125.19 47.02) (width 0.508) (layer "B.Cu") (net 10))
 (segment (start 127.73 62.255) (end 135.595 54.39) (width 0.508) (layer "B.Cu") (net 9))
 (segment (start 135.595 54.39) (end 148.33 54.39) (width 0.508) (layer "B.Cu") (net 9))
 (segment (start 148.33 54.39) (end 148.33 50.7556) (width 0.508) (layer "B.Cu") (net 9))
 (segment (start 149.04 46.25) (end 155.65 39.64) (width 0.508) (layer "B.Cu") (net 9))
 (segment (start 148.33 50.7556) (end 149.04 50.0456) (width 0.508) (layer "B.Cu") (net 9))
 (segment (start 149.04 50.0456) (end 149.04 46.25) (width 0.508) (layer "B.Cu") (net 9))
 (segment (start 143.26 57.11) (end 151.91 57.11) (width 0.508) (layer "B.Cu") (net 7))
 (segment (start 134.2704 60.7946) (end 134.2704 60.2296) (width 0.508) (layer "B.Cu") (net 7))
 (segment (start 151.91 57.11) (end 151.91 48.46) (width 0.508) (layer "B.Cu") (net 7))
 (segment (start 132.81 62.255) (end 134.2704 60.7946) (width 0.508) (layer "B.Cu") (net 7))
 (segment (start 134.2704 60.2296) (end 136.03 58.47) (width 0.508) (layer "B.Cu") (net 7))
 (segment (start 141.9 58.47) (end 143.26 57.11) (width 0.508) (layer "B.Cu") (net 7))
 (segment (start 136.03 58.47) (end 141.9 58.47) (width 0.508) (layer "B.Cu") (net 7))
 (segment (start 151.91 48.46) (end 155.65 44.72) (width 0.508) (layer "B.Cu") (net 7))
 (segment (start 147.342081 48.255) (end 147.82 47.777081) (width 0.508) (layer "B.Cu") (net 11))
 (segment (start 146.14 48.255) (end 147.342081 48.255) (width 0.508) (layer "B.Cu") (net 11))
 (segment (start 147.82 47.777081) (end 147.82 41.375) (width 0.508) (layer "B.Cu") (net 11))
 (segment (start 135.35 47.02) (end 135.35 44.89) (width 0.508) (layer "B.Cu") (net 15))
 (segment (start 135.35 44.89) (end 138.66 41.58) (width 0.508) (layer "B.Cu") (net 15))
 (segment (start 143.7196 36.9696) (end 145.34 38.59) (width 0.508) (layer "F.Cu") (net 19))
 (segment (start 126.01 38.78) (end 127.8204 36.9696) (width 0.508) (layer "F.Cu") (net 19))
 (segment (start 127.8204 36.9696) (end 143.7196 36.9696) (width 0.508) (layer "F.Cu") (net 19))
 (via (at 126.01 38.78) (size 1.6) (drill 0.86) (layers "F.Cu" "B.Cu") (free yes) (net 19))
 (via (at 145.34 38.59) (size 1.6) (drill 0.86) (layers "F.Cu" "B.Cu") (free yes) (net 19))
 (segment (start 125.96 38.83) (end 126.01 38.78) (width 0.508) (layer "B.Cu") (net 19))
 (segment (start 145.28 41.375) (end 145.28 38.65) (width 0.508) (layer "B.Cu") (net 19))
 (segment (start 145.28 38.65) (end 145.34 38.59) (width 0.508) (layer "B.Cu") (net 19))
 (segment (start 125.96 41.58) (end 125.96 38.83) (width 0.508) (layer "B.Cu") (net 19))
 (segment (start 132.81 45.89) (end 132.81 47.02) (width 0.508) (layer "B.Cu") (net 16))
 (segment (start 128.5 41.58) (end 132.81 45.89) (width 0.508) (layer "B.Cu") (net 16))
 (segment (start 137.89 47.02) (end 140.1704 44.7396) (width 0.508) (layer "B.Cu") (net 14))
 (segment (start 135.0904 40.0696) (end 133.58 41.58) (width 0.508) (layer "B.Cu") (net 14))
 (segment (start 140.1704 44.7396) (end 140.1704 40.4104) (width 0.508) (layer "B.Cu") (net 14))
 (segment (start 140.1704 40.4104) (end 139.8296 40.0696) (width 0.508) (layer "B.Cu") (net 14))
 (segment (start 139.8296 40.0696) (end 135.0904 40.0696) (width 0.508) (layer "B.Cu") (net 14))
 (segment (start 152.502 63.328) (end 152.33 63.5) (width 0.508) (layer "F.Cu") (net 17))
 (segment (start 156.496 63.328) (end 152.502 63.328) (width 0.508) (layer "F.Cu") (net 17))
 (via (at 152.33 63.5) (size 1.6) (drill 0.86) (layers "F.Cu" "B.Cu") (free yes) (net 17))
 (segment (start 152.33 63.5) (end 149.33 63.5) (width 0.508) (layer "B.Cu") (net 17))
 (segment (start 152.778 61.328) (end 152.4 60.95) (width 0.508) (layer "F.Cu") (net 18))
 (segment (start 156.496 61.328) (end 152.778 61.328) (width 0.508) (layer "F.Cu") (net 18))
 (via (at 152.4 60.95) (size 1.6) (drill 0.86) (layers "F.Cu" "B.Cu") (free yes) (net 18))
 (segment (start 152.4 60.95) (end 149.32 60.95) (width 0.508) (layer "B.Cu") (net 18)))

